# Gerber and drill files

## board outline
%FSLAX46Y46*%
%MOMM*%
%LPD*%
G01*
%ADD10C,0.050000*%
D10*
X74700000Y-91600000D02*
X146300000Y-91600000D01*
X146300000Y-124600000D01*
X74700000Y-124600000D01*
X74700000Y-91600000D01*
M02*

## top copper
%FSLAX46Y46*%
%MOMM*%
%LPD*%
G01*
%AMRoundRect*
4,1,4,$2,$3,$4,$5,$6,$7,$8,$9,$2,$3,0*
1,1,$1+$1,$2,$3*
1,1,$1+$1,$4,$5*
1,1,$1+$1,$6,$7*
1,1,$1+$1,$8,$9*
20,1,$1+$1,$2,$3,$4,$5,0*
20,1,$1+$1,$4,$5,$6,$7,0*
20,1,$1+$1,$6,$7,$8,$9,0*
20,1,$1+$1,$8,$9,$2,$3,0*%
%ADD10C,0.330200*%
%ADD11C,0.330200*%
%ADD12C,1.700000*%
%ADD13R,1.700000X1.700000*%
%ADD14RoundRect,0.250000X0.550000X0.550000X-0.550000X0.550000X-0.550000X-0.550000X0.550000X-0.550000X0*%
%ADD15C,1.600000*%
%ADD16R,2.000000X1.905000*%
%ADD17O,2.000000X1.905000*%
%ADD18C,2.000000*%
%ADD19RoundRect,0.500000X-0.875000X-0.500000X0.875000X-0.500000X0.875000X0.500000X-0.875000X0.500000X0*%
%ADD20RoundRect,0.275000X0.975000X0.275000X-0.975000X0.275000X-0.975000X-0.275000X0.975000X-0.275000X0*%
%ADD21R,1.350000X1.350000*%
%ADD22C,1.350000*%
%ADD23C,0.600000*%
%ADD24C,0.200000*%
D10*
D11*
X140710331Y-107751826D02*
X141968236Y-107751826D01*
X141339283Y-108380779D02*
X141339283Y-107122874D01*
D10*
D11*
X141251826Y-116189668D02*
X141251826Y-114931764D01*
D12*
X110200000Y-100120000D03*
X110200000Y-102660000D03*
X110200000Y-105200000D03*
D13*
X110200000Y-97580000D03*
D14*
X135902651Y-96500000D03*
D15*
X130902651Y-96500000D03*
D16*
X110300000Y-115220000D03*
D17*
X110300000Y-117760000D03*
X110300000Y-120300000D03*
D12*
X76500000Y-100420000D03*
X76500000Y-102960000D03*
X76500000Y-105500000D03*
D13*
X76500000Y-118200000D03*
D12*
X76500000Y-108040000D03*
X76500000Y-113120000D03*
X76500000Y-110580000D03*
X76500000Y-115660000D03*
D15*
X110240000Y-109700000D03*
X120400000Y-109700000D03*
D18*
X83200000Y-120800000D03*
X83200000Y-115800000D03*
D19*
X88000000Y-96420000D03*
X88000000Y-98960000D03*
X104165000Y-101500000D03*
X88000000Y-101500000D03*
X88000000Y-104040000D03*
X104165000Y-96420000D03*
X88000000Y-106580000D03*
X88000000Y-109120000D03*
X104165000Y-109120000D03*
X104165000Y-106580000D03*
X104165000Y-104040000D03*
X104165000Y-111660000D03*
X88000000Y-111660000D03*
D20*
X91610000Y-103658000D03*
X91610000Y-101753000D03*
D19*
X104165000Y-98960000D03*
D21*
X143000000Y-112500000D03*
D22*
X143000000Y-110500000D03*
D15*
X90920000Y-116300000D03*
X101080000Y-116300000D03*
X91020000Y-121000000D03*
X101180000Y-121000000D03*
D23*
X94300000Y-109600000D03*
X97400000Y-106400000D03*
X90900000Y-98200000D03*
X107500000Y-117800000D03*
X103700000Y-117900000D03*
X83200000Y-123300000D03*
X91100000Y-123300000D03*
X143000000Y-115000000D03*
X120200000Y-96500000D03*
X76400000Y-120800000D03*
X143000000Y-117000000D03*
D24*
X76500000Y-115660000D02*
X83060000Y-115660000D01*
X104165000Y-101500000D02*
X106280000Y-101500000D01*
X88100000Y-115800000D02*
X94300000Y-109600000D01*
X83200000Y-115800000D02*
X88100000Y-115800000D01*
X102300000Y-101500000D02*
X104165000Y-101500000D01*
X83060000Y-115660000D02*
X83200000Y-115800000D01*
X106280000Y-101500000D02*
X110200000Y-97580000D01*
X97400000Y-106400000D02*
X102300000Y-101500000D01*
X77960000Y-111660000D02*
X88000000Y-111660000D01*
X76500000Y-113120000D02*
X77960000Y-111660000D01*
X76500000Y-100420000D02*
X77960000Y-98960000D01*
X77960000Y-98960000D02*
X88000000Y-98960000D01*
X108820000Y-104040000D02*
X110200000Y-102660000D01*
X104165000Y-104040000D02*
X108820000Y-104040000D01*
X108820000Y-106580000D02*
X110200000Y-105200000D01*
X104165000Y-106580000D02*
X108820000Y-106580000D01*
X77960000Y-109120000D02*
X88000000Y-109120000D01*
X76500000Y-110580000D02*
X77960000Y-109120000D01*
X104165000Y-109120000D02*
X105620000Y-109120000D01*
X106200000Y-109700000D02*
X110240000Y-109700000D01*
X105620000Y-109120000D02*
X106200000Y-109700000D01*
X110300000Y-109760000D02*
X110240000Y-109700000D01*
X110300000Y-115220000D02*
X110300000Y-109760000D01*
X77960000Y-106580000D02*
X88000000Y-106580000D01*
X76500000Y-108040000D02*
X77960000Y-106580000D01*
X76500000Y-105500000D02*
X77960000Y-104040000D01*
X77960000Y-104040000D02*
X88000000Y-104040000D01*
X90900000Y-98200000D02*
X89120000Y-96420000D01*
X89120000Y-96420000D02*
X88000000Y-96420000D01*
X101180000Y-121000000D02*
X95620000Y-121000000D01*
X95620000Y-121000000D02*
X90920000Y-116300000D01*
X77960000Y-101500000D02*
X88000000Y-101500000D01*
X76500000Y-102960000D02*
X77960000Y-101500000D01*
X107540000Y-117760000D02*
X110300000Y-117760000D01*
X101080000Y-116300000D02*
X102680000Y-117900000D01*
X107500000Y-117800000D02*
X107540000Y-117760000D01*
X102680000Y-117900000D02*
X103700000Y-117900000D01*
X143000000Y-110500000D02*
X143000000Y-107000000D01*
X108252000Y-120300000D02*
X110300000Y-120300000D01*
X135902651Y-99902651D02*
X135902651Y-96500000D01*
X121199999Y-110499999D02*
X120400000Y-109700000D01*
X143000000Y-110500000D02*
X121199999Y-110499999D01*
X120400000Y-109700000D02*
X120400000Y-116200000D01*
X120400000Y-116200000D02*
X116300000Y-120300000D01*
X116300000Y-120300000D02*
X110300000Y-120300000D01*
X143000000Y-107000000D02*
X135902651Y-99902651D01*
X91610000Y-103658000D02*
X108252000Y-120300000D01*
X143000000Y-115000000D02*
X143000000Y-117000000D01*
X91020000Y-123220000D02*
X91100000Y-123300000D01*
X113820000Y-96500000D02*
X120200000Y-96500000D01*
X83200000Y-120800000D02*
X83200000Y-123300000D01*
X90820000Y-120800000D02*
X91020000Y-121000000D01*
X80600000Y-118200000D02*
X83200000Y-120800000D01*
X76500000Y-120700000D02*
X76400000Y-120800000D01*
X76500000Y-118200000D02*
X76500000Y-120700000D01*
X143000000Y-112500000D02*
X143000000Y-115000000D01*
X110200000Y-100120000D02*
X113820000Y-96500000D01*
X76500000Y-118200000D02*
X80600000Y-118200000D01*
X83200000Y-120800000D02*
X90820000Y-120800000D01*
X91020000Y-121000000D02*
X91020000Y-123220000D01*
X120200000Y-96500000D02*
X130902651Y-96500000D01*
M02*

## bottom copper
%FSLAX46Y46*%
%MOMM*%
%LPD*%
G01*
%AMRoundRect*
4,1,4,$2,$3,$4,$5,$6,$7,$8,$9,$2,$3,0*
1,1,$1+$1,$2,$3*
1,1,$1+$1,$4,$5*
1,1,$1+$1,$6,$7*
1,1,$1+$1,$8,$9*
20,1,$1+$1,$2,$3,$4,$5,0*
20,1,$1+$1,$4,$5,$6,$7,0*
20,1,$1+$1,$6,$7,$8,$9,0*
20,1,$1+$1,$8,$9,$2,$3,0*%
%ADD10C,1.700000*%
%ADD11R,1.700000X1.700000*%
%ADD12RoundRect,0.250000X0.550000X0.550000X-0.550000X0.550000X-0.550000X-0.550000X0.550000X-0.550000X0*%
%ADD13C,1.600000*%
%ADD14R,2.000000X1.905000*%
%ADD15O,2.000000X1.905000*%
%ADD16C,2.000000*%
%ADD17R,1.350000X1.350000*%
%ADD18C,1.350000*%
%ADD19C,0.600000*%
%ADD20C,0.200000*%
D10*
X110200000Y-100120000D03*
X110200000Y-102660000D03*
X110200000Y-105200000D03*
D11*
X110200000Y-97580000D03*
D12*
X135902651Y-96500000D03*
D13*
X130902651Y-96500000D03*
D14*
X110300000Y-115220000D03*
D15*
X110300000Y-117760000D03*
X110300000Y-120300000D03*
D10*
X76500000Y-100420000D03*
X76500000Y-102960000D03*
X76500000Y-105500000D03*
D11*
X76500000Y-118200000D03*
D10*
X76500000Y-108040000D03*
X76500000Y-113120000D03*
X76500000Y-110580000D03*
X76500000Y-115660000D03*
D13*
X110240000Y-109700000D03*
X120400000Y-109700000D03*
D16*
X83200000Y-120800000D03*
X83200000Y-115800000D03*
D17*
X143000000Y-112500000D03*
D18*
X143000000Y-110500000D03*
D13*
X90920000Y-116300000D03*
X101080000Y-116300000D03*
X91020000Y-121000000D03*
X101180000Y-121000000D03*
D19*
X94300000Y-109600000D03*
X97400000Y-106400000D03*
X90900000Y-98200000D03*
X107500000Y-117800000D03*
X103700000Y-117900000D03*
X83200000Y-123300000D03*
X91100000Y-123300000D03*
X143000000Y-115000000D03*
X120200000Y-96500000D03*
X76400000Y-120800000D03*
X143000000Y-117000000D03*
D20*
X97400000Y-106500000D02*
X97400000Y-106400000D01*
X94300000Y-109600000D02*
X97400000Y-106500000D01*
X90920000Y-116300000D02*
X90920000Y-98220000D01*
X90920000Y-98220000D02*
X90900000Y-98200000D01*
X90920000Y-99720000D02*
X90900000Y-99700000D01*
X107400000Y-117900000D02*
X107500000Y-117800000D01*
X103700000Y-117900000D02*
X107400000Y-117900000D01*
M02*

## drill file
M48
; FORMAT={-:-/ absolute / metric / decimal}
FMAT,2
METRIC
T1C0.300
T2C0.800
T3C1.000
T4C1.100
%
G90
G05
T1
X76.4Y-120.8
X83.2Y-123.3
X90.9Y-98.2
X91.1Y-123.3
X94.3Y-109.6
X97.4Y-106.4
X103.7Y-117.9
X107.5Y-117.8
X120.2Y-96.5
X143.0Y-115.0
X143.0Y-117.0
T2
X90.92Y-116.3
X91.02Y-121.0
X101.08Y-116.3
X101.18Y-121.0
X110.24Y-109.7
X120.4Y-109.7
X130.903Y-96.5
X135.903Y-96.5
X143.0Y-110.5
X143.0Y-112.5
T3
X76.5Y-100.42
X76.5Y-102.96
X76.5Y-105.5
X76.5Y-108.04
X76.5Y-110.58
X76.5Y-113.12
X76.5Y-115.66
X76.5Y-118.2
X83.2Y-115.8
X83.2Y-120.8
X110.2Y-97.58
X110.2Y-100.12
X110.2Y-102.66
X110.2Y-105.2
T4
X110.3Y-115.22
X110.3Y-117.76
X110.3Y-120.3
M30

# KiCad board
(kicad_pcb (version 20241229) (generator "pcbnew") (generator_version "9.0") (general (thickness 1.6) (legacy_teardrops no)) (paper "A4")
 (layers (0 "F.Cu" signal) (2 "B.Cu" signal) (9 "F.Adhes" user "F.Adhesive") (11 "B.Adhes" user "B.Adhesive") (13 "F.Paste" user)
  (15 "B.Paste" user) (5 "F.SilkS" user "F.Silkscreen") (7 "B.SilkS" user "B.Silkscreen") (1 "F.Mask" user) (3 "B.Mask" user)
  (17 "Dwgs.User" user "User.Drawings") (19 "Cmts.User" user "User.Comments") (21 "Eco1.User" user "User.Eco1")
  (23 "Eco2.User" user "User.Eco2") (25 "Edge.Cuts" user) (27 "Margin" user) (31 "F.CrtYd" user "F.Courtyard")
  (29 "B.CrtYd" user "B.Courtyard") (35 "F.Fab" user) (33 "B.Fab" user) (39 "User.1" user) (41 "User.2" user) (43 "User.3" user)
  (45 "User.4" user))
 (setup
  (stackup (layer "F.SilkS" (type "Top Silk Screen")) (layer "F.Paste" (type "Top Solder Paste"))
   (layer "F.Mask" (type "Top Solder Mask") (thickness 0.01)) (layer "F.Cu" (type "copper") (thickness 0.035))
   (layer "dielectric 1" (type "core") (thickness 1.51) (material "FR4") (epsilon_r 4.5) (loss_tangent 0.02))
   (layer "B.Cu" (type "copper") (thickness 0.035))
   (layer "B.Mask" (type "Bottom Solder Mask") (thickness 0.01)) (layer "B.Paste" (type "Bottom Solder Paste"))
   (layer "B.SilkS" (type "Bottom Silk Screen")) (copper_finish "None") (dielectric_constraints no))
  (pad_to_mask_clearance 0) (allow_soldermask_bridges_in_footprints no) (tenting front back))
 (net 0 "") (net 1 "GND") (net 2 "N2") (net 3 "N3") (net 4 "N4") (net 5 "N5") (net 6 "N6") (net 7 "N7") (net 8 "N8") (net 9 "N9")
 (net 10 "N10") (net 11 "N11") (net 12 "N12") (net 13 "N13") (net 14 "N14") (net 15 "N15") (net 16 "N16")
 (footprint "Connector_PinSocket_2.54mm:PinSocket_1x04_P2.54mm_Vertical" (layer "F.Cu") (at 110.2 97.58)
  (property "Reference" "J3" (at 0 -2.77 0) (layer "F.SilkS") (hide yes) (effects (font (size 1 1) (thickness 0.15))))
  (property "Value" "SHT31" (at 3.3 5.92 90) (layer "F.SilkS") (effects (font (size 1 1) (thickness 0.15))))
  (pad "GND" thru_hole circle (at 0 2.54) (size 1.7 1.7) (drill 1) (layers "*.Cu" "*.Mask") (remove_unused_layers no) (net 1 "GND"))
  (pad "SCL" thru_hole circle (at 0 5.08) (size 1.7 1.7) (drill 1) (layers "*.Cu" "*.Mask") (remove_unused_layers no) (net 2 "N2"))
  (pad "SDA" thru_hole circle (at 0 7.62) (size 1.7 1.7) (drill 1) (layers "*.Cu" "*.Mask") (remove_unused_layers no) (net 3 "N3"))
  (pad "VIN" thru_hole rect (at 0 0) (size 1.7 1.7) (drill 1) (layers "*.Cu" "*.Mask") (remove_unused_layers no) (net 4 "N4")))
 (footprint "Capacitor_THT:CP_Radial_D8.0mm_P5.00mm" (layer "F.Cu") (at 135.902651 96.5 180)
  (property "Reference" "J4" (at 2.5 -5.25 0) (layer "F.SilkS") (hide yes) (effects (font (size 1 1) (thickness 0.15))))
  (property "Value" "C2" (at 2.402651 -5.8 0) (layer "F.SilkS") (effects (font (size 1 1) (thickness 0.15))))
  (pad "+" thru_hole roundrect (at 0 0 180) (size 1.6 1.6) (drill 0.8) (layers "*.Cu" "*.Mask") (remove_unused_layers no)
   (roundrect_rratio 0.15625) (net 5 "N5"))
  (pad "-" thru_hole circle (at 5 0 180) (size 1.6 1.6) (drill 0.8) (layers "*.Cu" "*.Mask") (remove_unused_layers no) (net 1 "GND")))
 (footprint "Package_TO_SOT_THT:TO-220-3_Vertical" (layer "F.Cu") (at 110.3 115.22 -90)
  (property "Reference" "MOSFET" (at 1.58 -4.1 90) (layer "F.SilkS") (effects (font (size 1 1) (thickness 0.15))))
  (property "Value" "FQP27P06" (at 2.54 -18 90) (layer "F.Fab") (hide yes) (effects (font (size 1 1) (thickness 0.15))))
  (pad "1" thru_hole rect (at 0 0 270) (size 1.905 2) (drill 1.1) (layers "*.Cu" "*.Mask") (remove_unused_layers no) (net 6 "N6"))
  (pad "2" thru_hole oval (at 2.54 0 270) (size 1.905 2) (drill 1.1) (layers "*.Cu" "*.Mask") (remove_unused_layers no) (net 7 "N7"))
  (pad "3" thru_hole oval (at 5.08 0 270) (size 1.905 2) (drill 1.1) (layers "*.Cu" "*.Mask") (remove_unused_layers no) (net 5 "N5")))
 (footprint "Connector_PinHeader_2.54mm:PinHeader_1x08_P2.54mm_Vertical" (layer "F.Cu") (at 76.5 118.2 180)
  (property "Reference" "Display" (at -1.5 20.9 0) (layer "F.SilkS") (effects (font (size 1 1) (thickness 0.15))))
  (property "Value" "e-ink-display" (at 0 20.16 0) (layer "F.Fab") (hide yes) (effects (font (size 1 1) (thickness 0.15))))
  (pad "BUSY" thru_hole circle (at 0 17.78 180) (size 1.7 1.7) (drill 1) (layers "*.Cu" "*.Mask") (remove_unused_layers no) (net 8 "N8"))
  (pad "CS" thru_hole circle (at 0 15.24 180) (size 1.7 1.7) (drill 1) (layers "*.Cu" "*.Mask") (remove_unused_layers no) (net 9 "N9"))
  (pad "DC" thru_hole circle (at 0 12.7 180) (size 1.7 1.7) (drill 1) (layers "*.Cu" "*.Mask") (remove_unused_layers no) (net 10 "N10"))
  (pad "GND" thru_hole rect (at 0 0 180) (size 1.7 1.7) (drill 1) (layers "*.Cu" "*.Mask") (remove_unused_layers no) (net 1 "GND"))
  (pad "RES" thru_hole circle (at 0 10.16 180) (size 1.7 1.7) (drill 1) (layers "*.Cu" "*.Mask") (remove_unused_layers no) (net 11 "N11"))
  (pad "SCL" thru_hole circle (at 0 5.08 180) (size 1.7 1.7) (drill 1) (layers "*.Cu" "*.Mask") (remove_unused_layers no) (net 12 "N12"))
  (pad "SDA" thru_hole circle (at 0 7.62 180) (size 1.7 1.7) (drill 1) (layers "*.Cu" "*.Mask") (remove_unused_layers no) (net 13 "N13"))
  (pad "VCC" thru_hole circle (at 0 2.54 180) (size 1.7 1.7) (drill 1) (layers "*.Cu" "*.Mask") (remove_unused_layers no) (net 4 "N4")))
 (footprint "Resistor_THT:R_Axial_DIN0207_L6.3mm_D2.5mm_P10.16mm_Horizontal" (layer "F.Cu") (at 110.24 109.7)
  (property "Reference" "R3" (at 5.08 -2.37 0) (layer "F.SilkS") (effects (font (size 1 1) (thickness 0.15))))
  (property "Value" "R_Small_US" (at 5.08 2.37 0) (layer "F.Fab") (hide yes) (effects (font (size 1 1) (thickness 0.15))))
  (pad "1" thru_hole circle (at 0 0) (size 1.6 1.6) (drill 0.8) (layers "*.Cu" "*.Mask") (remove_unused_layers no) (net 6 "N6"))
  (pad "2" thru_hole circle (at 10.16 0) (size 1.6 1.6) (drill 0.8) (layers "*.Cu" "*.Mask") (remove_unused_layers no) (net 5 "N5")))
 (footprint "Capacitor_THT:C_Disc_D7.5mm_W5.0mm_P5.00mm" (layer "F.Cu") (at 83.2 120.8 90)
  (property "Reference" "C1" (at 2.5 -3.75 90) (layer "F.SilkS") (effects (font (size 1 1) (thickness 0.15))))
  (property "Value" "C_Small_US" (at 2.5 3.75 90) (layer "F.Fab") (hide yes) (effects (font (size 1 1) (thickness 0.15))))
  (pad "1" thru_hole circle (at 0 0 90) (size 2 2) (drill 1) (layers "*.Cu" "*.Mask") (remove_unused_layers no) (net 1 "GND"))
  (pad "2" thru_hole circle (at 5 0 90) (size 2 2) (drill 1) (layers "*.Cu" "*.Mask") (remove_unused_layers no) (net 4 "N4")))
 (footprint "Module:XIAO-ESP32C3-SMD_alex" (layer "F.Cu") (at 96 104)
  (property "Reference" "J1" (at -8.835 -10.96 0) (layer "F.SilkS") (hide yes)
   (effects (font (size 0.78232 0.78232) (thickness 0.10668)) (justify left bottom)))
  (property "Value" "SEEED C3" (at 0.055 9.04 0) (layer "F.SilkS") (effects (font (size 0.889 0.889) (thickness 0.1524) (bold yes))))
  (pad "2" smd roundrect (at -8 -7.58) (size 2.75 2) (layers "F.Cu" "F.Mask" "F.Paste") (roundrect_rratio 0.25) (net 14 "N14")
   (solder_mask_margin 0.0508) (thermal_bridge_angle 45))
  (pad "3" smd roundrect (at -8 -5.04) (size 2.75 2) (layers "F.Cu" "F.Mask" "F.Paste") (roundrect_rratio 0.25) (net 8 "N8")
   (solder_mask_margin 0.0508) (thermal_bridge_angle 45))
  (pad "3.3V" smd roundrect (at 8.165 -2.5) (size 2.75 2) (layers "F.Cu" "F.Mask" "F.Paste") (roundrect_rratio 0.25) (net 4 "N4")
   (solder_mask_margin 0.0508) (thermal_bridge_angle 45))
  (pad "4" smd roundrect (at -8 -2.5) (size 2.75 2) (layers "F.Cu" "F.Mask" "F.Paste") (roundrect_rratio 0.25) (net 9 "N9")
   (solder_mask_margin 0.0508) (thermal_bridge_angle 45))
  (pad "5" smd roundrect (at -8 0.04) (size 2.75 2) (layers "F.Cu" "F.Mask" "F.Paste") (roundrect_rratio 0.25) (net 10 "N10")
   (solder_mask_margin 0.0508) (thermal_bridge_angle 45))
  (pad "5V" smd roundrect (at 8.165 -7.58) (size 2.75 2) (layers "F.Cu" "F.Mask" "F.Paste") (roundrect_rratio 0.25) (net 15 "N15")
   (solder_mask_margin 0.0508) (thermal_bridge_angle 45))
  (pad "6" smd roundrect (at -8 2.58) (size 2.75 2) (layers "F.Cu" "F.Mask" "F.Paste") (roundrect_rratio 0.25) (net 11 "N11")
   (solder_mask_margin 0.0508) (thermal_bridge_angle 45))
  (pad "7" smd roundrect (at -8 5.12) (size 2.75 2) (layers "F.Cu" "F.Mask" "F.Paste") (roundrect_rratio 0.25) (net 13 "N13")
   (solder_mask_margin 0.0508) (thermal_bridge_angle 45))
  (pad "8" smd roundrect (at 8.165 5.12) (size 2.75 2) (layers "F.Cu" "F.Mask" "F.Paste") (roundrect_rratio 0.25) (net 6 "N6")
   (solder_mask_margin 0.0508) (thermal_bridge_angle 45))
  (pad "9" smd roundrect (at 8.165 2.58) (size 2.75 2) (layers "F.Cu" "F.Mask" "F.Paste") (roundrect_rratio 0.25) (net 3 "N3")
   (solder_mask_margin 0.0508) (thermal_bridge_angle 45))
  (pad "10" smd roundrect (at 8.165 0.04) (size 2.75 2) (layers "F.Cu" "F.Mask" "F.Paste") (roundrect_rratio 0.25) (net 2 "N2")
   (solder_mask_margin 0.0508) (thermal_bridge_angle 45))
  (pad "20" smd roundrect (at 8.165 7.66) (size 2.75 2) (layers "F.Cu" "F.Mask" "F.Paste") (roundrect_rratio 0.25) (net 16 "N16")
   (solder_mask_margin 0.0508) (thermal_bridge_angle 45))
  (pad "21" smd roundrect (at -8 7.66) (size 2.75 2) (layers "F.Cu" "F.Mask" "F.Paste") (roundrect_rratio 0.25) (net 12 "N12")
   (solder_mask_margin 0.0508) (thermal_bridge_angle 45))
  (pad "BAT+" smd roundrect (at -4.39 -0.342 180) (size 2.5 1.1) (layers "F.Cu" "F.Mask" "F.Paste") (roundrect_rratio 0.25) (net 5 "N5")
   (solder_mask_margin 0.0508) (thermal_bridge_angle 45))
  (pad "BAT-" smd roundrect (at -4.39 -2.247 180) (size 2.5 1.1) (layers "F.Cu" "F.Mask" "F.Paste") (roundrect_rratio 0.25) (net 1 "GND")
   (solder_mask_margin 0.0508) (thermal_bridge_angle 45))
  (pad "GND" smd roundrect (at 8.165 -5.04) (size 2.75 2) (layers "F.Cu" "F.Mask" "F.Paste") (roundrect_rratio 0.25) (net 1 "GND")
   (solder_mask_margin 0.0508) (thermal_bridge_angle 45)))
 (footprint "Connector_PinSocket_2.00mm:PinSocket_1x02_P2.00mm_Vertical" (layer "F.Cu") (at 143 112.5 180)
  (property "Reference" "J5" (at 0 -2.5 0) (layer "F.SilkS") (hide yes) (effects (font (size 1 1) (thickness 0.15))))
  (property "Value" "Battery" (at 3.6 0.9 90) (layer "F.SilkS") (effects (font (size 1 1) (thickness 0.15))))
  (pad "1" thru_hole rect (at 0 0 180) (size 1.35 1.35) (drill 0.8) (layers "*.Cu" "*.Mask") (remove_unused_layers no) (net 1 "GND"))
  (pad "2" thru_hole circle (at 0 2 180) (size 1.35 1.35) (drill 0.8) (layers "*.Cu" "*.Mask") (remove_unused_layers no) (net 5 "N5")))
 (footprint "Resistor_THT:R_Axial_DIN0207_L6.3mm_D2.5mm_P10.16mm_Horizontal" (layer "F.Cu") (at 90.92 116.3)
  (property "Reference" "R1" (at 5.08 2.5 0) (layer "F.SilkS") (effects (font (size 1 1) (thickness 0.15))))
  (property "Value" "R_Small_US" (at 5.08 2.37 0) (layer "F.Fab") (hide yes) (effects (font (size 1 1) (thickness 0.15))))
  (pad "1" thru_hole circle (at 0 0) (size 1.6 1.6) (drill 0.8) (layers "*.Cu" "*.Mask") (remove_unused_layers no) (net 14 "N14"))
  (pad "2" thru_hole circle (at 10.16 0) (size 1.6 1.6) (drill 0.8) (layers "*.Cu" "*.Mask") (remove_unused_layers no) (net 7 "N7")))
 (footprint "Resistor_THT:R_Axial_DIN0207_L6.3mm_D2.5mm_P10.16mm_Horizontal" (layer "F.Cu") (at 91.02 121)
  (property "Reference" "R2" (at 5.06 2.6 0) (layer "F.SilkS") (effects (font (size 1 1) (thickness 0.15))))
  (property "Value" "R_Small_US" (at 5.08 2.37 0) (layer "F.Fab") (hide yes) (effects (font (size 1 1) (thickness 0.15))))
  (pad "1" thru_hole circle (at 0 0) (size 1.6 1.6) (drill 0.8) (layers "*.Cu" "*.Mask") (remove_unused_layers no) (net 1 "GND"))
  (pad "2" thru_hole circle (at 10.16 0) (size 1.6 1.6) (drill 0.8) (layers "*.Cu" "*.Mask") (remove_unused_layers no) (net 14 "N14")))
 (gr_rect (start 74.7 91.6) (end 146.3 124.6) (stroke (width 0.05) (type solid)) (fill no) (layer "Edge.Cuts"))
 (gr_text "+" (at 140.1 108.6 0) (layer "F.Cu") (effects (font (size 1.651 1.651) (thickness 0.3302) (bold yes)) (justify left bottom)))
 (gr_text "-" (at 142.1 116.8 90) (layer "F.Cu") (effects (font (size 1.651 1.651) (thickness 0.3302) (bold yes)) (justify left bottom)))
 (segment (start 76.5 115.66) (end 83.06 115.66) (width 0.2) (layer "F.Cu") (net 4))
 (segment (start 104.165 101.5) (end 106.28 101.5) (width 0.2) (layer "F.Cu") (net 4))
 (segment (start 88.1 115.8) (end 94.3 109.6) (width 0.2) (layer "F.Cu") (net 4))
 (segment (start 83.2 115.8) (end 88.1 115.8) (width 0.2) (layer "F.Cu") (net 4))
 (segment (start 102.3 101.5) (end 104.165 101.5) (width 0.2) (layer "F.Cu") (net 4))
 (segment (start 83.06 115.66) (end 83.2 115.8) (width 0.2) (layer "F.Cu") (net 4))
 (segment (start 106.28 101.5) (end 110.2 97.58) (width 0.2) (layer "F.Cu") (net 4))
 (segment (start 97.4 106.4) (end 102.3 101.5) (width 0.2) (layer "F.Cu") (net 4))
 (via (at 94.3 109.6) (size 0.6) (drill 0.3) (layers "F.Cu" "B.Cu") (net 4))
 (via (at 97.4 106.4) (size 0.6) (drill 0.3) (layers "F.Cu" "B.Cu") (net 4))
 (segment (start 97.4 106.5) (end 97.4 106.4) (width 0.2) (layer "B.Cu") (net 4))
 (segment (start 94.3 109.6) (end 97.4 106.5) (width 0.2) (layer "B.Cu") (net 4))
 (segment (start 77.96 111.66) (end 88 111.66) (width 0.2) (layer "F.Cu") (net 12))
 (segment (start 76.5 113.12) (end 77.96 111.66) (width 0.2) (layer "F.Cu") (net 12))
 (segment (start 76.5 100.42) (end 77.96 98.96) (width 0.2) (layer "F.Cu") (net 8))
 (segment (start 77.96 98.96) (end 88 98.96) (width 0.2) (layer "F.Cu") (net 8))
 (segment (start 108.82 104.04) (end 110.2 102.66) (width 0.2) (layer "F.Cu") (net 2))
 (segment (start 104.165 104.04) (end 108.82 104.04) (width 0.2) (layer "F.Cu") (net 2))
 (segment (start 108.82 106.58) (end 110.2 105.2) (width 0.2) (layer "F.Cu") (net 3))
 (segment (start 104.165 106.58) (end 108.82 106.58) (width 0.2) (layer "F.Cu") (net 3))
 (segment (start 77.96 109.12) (end 88 109.12) (width 0.2) (layer "F.Cu") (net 13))
 (segment (start 76.5 110.58) (end 77.96 109.12) (width 0.2) (layer "F.Cu") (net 13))
 (segment (start 104.165 109.12) (end 105.62 109.12) (width 0.2) (layer "F.Cu") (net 6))
 (segment (start 106.2 109.7) (end 110.24 109.7) (width 0.2) (layer "F.Cu") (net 6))
 (segment (start 105.62 109.12) (end 106.2 109.7) (width 0.2) (layer "F.Cu") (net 6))
 (segment (start 110.3 109.76) (end 110.24 109.7) (width 0.2) (layer "F.Cu") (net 6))
 (segment (start 110.3 115.22) (end 110.3 109.76) (width 0.2) (layer "F.Cu") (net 6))
 (segment (start 77.96 106.58) (end 88 106.58) (width 0.2) (layer "F.Cu") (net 11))
 (segment (start 76.5 108.04) (end 77.96 106.58) (width 0.2) (layer "F.Cu") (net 11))
 (segment (start 76.5 105.5) (end 77.96 104.04) (width 0.2) (layer "F.Cu") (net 10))
 (segment (start 77.96 104.04) (end 88 104.04) (width 0.2) (layer "F.Cu") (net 10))
 (segment (start 90.9 98.2) (end 89.12 96.42) (width 0.2) (layer "F.Cu") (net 14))
 (segment (start 89.12 96.42) (end 88 96.42) (width 0.2) (layer "F.Cu") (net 14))
 (segment (start 101.18 121) (end 95.62 121) (width 0.2) (layer "F.Cu") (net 14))
 (segment (start 95.62 121) (end 90.92 116.3) (width 0.2) (layer "F.Cu") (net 14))
 (via (at 90.9 98.2) (size 0.6) (drill 0.3) (layers "F.Cu" "B.Cu") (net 14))
 (segment (start 90.92 116.3) (end 90.92 98.22) (width 0.2) (layer "B.Cu") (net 14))
 (segment (start 90.92 98.22) (end 90.9 98.2) (width 0.2) (layer "B.Cu") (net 14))
 (segment (start 90.92 99.72) (end 90.9 99.7) (width 0.2) (layer "B.Cu") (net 14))
 (segment (start 77.96 101.5) (end 88 101.5) (width 0.2) (layer "F.Cu") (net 9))
 (segment (start 76.5 102.96) (end 77.96 101.5) (width 0.2) (layer "F.Cu") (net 9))
 (segment (start 107.54 117.76) (end 110.3 117.76) (width 0.2) (layer "F.Cu") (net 7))
 (segment (start 101.08 116.3) (end 102.68 117.9) (width 0.2) (layer "F.Cu") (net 7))
 (segment (start 107.5 117.8) (end 107.54 117.76) (width 0.2) (layer "F.Cu") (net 7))
 (segment (start 102.68 117.9) (end 103.7 117.9) (width 0.2) (layer "F.Cu") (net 7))
 (via (at 107.5 117.8) (size 0.6) (drill 0.3) (layers "F.Cu" "B.Cu") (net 7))
 (via (at 103.7 117.9) (size 0.6) (drill 0.3) (layers "F.Cu" "B.Cu") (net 7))
 (segment (start 107.4 117.9) (end 107.5 117.8) (width 0.2) (layer "B.Cu") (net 7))
 (segment (start 103.7 117.9) (end 107.4 117.9) (width 0.2) (layer "B.Cu") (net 7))
 (segment (start 143 110.5) (end 143 107) (width 0.2) (layer "F.Cu") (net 5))
 (segment (start 108.252 120.3) (end 110.3 120.3) (width 0.2) (layer "F.Cu") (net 5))
 (segment (start 135.902651 99.902651) (end 135.902651 96.5) (width 0.2) (layer "F.Cu") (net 5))
 (segment (start 121.199999 110.499999) (end 120.4 109.7) (width 0.2) (layer "F.Cu") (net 5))
 (segment (start 143 110.5) (end 121.199999 110.499999) (width 0.2) (layer "F.Cu") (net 5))
 (segment (start 120.4 109.7) (end 120.4 116.2) (width 0.2) (layer "F.Cu") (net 5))
 (segment (start 120.4 116.2) (end 116.3 120.3) (width 0.2) (layer "F.Cu") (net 5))
 (segment (start 116.3 120.3) (end 110.3 120.3) (width 0.2) (layer "F.Cu") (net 5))
 (segment (start 143 107) (end 135.902651 99.902651) (width 0.2) (layer "F.Cu") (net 5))
 (segment (start 91.61 103.658) (end 108.252 120.3) (width 0.2) (layer "F.Cu") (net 5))
 (segment (start 143 115) (end 143 117) (width 0.2) (layer "F.Cu") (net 1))
 (segment (start 91.02 123.22) (end 91.1 123.3) (width 0.2) (layer "F.Cu") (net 1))
 (segment (start 113.82 96.5) (end 120.2 96.5) (width 0.2) (layer "F.Cu") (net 1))
 (segment (start 83.2 120.8) (end 83.2 123.3) (width 0.2) (layer "F.Cu") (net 1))
 (segment (start 90.82 120.8) (end 91.02 121) (width 0.2) (layer "F.Cu") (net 1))
 (segment (start 80.6 118.2) (end 83.2 120.8) (width 0.2) (layer "F.Cu") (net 1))
 (segment (start 76.5 120.7) (end 76.4 120.8) (width 0.2) (layer "F.Cu") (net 1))
 (segment (start 76.5 118.2) (end 76.5 120.7) (width 0.2) (layer "F.Cu") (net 1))
 (segment (start 143 112.5) (end 143 115) (width 0.2) (layer "F.Cu") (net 1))
 (segment (start 110.2 100.12) (end 113.82 96.5) (width 0.2) (layer "F.Cu") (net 1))
 (segment (start 76.5 118.2) (end 80.6 118.2) (width 0.2) (layer "F.Cu") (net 1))
 (segment (start 83.2 120.8) (end 90.82 120.8) (width 0.2) (layer "F.Cu") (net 1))
 (segment (start 91.02 121) (end 91.02 123.22) (width 0.2) (layer "F.Cu") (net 1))
 (segment (start 120.2 96.5) (end 130.902651 96.5) (width 0.2) (layer "F.Cu") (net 1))
 (via (at 83.2 123.3) (size 0.6) (drill 0.3) (layers "F.Cu" "B.Cu") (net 1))
 (via (at 91.1 123.3) (size 0.6) (drill 0.3) (layers "F.Cu" "B.Cu") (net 1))
 (via (at 143 115) (size 0.6) (drill 0.3) (layers "F.Cu" "B.Cu") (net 1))
 (via (at 120.2 96.5) (size 0.6) (drill 0.3) (layers "F.Cu" "B.Cu") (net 1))
 (via (at 76.4 120.8) (size 0.6) (drill 0.3) (layers "F.Cu" "B.Cu") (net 1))
 (via (at 143 117) (size 0.6) (drill 0.3) (layers "F.Cu" "B.Cu") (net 1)))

